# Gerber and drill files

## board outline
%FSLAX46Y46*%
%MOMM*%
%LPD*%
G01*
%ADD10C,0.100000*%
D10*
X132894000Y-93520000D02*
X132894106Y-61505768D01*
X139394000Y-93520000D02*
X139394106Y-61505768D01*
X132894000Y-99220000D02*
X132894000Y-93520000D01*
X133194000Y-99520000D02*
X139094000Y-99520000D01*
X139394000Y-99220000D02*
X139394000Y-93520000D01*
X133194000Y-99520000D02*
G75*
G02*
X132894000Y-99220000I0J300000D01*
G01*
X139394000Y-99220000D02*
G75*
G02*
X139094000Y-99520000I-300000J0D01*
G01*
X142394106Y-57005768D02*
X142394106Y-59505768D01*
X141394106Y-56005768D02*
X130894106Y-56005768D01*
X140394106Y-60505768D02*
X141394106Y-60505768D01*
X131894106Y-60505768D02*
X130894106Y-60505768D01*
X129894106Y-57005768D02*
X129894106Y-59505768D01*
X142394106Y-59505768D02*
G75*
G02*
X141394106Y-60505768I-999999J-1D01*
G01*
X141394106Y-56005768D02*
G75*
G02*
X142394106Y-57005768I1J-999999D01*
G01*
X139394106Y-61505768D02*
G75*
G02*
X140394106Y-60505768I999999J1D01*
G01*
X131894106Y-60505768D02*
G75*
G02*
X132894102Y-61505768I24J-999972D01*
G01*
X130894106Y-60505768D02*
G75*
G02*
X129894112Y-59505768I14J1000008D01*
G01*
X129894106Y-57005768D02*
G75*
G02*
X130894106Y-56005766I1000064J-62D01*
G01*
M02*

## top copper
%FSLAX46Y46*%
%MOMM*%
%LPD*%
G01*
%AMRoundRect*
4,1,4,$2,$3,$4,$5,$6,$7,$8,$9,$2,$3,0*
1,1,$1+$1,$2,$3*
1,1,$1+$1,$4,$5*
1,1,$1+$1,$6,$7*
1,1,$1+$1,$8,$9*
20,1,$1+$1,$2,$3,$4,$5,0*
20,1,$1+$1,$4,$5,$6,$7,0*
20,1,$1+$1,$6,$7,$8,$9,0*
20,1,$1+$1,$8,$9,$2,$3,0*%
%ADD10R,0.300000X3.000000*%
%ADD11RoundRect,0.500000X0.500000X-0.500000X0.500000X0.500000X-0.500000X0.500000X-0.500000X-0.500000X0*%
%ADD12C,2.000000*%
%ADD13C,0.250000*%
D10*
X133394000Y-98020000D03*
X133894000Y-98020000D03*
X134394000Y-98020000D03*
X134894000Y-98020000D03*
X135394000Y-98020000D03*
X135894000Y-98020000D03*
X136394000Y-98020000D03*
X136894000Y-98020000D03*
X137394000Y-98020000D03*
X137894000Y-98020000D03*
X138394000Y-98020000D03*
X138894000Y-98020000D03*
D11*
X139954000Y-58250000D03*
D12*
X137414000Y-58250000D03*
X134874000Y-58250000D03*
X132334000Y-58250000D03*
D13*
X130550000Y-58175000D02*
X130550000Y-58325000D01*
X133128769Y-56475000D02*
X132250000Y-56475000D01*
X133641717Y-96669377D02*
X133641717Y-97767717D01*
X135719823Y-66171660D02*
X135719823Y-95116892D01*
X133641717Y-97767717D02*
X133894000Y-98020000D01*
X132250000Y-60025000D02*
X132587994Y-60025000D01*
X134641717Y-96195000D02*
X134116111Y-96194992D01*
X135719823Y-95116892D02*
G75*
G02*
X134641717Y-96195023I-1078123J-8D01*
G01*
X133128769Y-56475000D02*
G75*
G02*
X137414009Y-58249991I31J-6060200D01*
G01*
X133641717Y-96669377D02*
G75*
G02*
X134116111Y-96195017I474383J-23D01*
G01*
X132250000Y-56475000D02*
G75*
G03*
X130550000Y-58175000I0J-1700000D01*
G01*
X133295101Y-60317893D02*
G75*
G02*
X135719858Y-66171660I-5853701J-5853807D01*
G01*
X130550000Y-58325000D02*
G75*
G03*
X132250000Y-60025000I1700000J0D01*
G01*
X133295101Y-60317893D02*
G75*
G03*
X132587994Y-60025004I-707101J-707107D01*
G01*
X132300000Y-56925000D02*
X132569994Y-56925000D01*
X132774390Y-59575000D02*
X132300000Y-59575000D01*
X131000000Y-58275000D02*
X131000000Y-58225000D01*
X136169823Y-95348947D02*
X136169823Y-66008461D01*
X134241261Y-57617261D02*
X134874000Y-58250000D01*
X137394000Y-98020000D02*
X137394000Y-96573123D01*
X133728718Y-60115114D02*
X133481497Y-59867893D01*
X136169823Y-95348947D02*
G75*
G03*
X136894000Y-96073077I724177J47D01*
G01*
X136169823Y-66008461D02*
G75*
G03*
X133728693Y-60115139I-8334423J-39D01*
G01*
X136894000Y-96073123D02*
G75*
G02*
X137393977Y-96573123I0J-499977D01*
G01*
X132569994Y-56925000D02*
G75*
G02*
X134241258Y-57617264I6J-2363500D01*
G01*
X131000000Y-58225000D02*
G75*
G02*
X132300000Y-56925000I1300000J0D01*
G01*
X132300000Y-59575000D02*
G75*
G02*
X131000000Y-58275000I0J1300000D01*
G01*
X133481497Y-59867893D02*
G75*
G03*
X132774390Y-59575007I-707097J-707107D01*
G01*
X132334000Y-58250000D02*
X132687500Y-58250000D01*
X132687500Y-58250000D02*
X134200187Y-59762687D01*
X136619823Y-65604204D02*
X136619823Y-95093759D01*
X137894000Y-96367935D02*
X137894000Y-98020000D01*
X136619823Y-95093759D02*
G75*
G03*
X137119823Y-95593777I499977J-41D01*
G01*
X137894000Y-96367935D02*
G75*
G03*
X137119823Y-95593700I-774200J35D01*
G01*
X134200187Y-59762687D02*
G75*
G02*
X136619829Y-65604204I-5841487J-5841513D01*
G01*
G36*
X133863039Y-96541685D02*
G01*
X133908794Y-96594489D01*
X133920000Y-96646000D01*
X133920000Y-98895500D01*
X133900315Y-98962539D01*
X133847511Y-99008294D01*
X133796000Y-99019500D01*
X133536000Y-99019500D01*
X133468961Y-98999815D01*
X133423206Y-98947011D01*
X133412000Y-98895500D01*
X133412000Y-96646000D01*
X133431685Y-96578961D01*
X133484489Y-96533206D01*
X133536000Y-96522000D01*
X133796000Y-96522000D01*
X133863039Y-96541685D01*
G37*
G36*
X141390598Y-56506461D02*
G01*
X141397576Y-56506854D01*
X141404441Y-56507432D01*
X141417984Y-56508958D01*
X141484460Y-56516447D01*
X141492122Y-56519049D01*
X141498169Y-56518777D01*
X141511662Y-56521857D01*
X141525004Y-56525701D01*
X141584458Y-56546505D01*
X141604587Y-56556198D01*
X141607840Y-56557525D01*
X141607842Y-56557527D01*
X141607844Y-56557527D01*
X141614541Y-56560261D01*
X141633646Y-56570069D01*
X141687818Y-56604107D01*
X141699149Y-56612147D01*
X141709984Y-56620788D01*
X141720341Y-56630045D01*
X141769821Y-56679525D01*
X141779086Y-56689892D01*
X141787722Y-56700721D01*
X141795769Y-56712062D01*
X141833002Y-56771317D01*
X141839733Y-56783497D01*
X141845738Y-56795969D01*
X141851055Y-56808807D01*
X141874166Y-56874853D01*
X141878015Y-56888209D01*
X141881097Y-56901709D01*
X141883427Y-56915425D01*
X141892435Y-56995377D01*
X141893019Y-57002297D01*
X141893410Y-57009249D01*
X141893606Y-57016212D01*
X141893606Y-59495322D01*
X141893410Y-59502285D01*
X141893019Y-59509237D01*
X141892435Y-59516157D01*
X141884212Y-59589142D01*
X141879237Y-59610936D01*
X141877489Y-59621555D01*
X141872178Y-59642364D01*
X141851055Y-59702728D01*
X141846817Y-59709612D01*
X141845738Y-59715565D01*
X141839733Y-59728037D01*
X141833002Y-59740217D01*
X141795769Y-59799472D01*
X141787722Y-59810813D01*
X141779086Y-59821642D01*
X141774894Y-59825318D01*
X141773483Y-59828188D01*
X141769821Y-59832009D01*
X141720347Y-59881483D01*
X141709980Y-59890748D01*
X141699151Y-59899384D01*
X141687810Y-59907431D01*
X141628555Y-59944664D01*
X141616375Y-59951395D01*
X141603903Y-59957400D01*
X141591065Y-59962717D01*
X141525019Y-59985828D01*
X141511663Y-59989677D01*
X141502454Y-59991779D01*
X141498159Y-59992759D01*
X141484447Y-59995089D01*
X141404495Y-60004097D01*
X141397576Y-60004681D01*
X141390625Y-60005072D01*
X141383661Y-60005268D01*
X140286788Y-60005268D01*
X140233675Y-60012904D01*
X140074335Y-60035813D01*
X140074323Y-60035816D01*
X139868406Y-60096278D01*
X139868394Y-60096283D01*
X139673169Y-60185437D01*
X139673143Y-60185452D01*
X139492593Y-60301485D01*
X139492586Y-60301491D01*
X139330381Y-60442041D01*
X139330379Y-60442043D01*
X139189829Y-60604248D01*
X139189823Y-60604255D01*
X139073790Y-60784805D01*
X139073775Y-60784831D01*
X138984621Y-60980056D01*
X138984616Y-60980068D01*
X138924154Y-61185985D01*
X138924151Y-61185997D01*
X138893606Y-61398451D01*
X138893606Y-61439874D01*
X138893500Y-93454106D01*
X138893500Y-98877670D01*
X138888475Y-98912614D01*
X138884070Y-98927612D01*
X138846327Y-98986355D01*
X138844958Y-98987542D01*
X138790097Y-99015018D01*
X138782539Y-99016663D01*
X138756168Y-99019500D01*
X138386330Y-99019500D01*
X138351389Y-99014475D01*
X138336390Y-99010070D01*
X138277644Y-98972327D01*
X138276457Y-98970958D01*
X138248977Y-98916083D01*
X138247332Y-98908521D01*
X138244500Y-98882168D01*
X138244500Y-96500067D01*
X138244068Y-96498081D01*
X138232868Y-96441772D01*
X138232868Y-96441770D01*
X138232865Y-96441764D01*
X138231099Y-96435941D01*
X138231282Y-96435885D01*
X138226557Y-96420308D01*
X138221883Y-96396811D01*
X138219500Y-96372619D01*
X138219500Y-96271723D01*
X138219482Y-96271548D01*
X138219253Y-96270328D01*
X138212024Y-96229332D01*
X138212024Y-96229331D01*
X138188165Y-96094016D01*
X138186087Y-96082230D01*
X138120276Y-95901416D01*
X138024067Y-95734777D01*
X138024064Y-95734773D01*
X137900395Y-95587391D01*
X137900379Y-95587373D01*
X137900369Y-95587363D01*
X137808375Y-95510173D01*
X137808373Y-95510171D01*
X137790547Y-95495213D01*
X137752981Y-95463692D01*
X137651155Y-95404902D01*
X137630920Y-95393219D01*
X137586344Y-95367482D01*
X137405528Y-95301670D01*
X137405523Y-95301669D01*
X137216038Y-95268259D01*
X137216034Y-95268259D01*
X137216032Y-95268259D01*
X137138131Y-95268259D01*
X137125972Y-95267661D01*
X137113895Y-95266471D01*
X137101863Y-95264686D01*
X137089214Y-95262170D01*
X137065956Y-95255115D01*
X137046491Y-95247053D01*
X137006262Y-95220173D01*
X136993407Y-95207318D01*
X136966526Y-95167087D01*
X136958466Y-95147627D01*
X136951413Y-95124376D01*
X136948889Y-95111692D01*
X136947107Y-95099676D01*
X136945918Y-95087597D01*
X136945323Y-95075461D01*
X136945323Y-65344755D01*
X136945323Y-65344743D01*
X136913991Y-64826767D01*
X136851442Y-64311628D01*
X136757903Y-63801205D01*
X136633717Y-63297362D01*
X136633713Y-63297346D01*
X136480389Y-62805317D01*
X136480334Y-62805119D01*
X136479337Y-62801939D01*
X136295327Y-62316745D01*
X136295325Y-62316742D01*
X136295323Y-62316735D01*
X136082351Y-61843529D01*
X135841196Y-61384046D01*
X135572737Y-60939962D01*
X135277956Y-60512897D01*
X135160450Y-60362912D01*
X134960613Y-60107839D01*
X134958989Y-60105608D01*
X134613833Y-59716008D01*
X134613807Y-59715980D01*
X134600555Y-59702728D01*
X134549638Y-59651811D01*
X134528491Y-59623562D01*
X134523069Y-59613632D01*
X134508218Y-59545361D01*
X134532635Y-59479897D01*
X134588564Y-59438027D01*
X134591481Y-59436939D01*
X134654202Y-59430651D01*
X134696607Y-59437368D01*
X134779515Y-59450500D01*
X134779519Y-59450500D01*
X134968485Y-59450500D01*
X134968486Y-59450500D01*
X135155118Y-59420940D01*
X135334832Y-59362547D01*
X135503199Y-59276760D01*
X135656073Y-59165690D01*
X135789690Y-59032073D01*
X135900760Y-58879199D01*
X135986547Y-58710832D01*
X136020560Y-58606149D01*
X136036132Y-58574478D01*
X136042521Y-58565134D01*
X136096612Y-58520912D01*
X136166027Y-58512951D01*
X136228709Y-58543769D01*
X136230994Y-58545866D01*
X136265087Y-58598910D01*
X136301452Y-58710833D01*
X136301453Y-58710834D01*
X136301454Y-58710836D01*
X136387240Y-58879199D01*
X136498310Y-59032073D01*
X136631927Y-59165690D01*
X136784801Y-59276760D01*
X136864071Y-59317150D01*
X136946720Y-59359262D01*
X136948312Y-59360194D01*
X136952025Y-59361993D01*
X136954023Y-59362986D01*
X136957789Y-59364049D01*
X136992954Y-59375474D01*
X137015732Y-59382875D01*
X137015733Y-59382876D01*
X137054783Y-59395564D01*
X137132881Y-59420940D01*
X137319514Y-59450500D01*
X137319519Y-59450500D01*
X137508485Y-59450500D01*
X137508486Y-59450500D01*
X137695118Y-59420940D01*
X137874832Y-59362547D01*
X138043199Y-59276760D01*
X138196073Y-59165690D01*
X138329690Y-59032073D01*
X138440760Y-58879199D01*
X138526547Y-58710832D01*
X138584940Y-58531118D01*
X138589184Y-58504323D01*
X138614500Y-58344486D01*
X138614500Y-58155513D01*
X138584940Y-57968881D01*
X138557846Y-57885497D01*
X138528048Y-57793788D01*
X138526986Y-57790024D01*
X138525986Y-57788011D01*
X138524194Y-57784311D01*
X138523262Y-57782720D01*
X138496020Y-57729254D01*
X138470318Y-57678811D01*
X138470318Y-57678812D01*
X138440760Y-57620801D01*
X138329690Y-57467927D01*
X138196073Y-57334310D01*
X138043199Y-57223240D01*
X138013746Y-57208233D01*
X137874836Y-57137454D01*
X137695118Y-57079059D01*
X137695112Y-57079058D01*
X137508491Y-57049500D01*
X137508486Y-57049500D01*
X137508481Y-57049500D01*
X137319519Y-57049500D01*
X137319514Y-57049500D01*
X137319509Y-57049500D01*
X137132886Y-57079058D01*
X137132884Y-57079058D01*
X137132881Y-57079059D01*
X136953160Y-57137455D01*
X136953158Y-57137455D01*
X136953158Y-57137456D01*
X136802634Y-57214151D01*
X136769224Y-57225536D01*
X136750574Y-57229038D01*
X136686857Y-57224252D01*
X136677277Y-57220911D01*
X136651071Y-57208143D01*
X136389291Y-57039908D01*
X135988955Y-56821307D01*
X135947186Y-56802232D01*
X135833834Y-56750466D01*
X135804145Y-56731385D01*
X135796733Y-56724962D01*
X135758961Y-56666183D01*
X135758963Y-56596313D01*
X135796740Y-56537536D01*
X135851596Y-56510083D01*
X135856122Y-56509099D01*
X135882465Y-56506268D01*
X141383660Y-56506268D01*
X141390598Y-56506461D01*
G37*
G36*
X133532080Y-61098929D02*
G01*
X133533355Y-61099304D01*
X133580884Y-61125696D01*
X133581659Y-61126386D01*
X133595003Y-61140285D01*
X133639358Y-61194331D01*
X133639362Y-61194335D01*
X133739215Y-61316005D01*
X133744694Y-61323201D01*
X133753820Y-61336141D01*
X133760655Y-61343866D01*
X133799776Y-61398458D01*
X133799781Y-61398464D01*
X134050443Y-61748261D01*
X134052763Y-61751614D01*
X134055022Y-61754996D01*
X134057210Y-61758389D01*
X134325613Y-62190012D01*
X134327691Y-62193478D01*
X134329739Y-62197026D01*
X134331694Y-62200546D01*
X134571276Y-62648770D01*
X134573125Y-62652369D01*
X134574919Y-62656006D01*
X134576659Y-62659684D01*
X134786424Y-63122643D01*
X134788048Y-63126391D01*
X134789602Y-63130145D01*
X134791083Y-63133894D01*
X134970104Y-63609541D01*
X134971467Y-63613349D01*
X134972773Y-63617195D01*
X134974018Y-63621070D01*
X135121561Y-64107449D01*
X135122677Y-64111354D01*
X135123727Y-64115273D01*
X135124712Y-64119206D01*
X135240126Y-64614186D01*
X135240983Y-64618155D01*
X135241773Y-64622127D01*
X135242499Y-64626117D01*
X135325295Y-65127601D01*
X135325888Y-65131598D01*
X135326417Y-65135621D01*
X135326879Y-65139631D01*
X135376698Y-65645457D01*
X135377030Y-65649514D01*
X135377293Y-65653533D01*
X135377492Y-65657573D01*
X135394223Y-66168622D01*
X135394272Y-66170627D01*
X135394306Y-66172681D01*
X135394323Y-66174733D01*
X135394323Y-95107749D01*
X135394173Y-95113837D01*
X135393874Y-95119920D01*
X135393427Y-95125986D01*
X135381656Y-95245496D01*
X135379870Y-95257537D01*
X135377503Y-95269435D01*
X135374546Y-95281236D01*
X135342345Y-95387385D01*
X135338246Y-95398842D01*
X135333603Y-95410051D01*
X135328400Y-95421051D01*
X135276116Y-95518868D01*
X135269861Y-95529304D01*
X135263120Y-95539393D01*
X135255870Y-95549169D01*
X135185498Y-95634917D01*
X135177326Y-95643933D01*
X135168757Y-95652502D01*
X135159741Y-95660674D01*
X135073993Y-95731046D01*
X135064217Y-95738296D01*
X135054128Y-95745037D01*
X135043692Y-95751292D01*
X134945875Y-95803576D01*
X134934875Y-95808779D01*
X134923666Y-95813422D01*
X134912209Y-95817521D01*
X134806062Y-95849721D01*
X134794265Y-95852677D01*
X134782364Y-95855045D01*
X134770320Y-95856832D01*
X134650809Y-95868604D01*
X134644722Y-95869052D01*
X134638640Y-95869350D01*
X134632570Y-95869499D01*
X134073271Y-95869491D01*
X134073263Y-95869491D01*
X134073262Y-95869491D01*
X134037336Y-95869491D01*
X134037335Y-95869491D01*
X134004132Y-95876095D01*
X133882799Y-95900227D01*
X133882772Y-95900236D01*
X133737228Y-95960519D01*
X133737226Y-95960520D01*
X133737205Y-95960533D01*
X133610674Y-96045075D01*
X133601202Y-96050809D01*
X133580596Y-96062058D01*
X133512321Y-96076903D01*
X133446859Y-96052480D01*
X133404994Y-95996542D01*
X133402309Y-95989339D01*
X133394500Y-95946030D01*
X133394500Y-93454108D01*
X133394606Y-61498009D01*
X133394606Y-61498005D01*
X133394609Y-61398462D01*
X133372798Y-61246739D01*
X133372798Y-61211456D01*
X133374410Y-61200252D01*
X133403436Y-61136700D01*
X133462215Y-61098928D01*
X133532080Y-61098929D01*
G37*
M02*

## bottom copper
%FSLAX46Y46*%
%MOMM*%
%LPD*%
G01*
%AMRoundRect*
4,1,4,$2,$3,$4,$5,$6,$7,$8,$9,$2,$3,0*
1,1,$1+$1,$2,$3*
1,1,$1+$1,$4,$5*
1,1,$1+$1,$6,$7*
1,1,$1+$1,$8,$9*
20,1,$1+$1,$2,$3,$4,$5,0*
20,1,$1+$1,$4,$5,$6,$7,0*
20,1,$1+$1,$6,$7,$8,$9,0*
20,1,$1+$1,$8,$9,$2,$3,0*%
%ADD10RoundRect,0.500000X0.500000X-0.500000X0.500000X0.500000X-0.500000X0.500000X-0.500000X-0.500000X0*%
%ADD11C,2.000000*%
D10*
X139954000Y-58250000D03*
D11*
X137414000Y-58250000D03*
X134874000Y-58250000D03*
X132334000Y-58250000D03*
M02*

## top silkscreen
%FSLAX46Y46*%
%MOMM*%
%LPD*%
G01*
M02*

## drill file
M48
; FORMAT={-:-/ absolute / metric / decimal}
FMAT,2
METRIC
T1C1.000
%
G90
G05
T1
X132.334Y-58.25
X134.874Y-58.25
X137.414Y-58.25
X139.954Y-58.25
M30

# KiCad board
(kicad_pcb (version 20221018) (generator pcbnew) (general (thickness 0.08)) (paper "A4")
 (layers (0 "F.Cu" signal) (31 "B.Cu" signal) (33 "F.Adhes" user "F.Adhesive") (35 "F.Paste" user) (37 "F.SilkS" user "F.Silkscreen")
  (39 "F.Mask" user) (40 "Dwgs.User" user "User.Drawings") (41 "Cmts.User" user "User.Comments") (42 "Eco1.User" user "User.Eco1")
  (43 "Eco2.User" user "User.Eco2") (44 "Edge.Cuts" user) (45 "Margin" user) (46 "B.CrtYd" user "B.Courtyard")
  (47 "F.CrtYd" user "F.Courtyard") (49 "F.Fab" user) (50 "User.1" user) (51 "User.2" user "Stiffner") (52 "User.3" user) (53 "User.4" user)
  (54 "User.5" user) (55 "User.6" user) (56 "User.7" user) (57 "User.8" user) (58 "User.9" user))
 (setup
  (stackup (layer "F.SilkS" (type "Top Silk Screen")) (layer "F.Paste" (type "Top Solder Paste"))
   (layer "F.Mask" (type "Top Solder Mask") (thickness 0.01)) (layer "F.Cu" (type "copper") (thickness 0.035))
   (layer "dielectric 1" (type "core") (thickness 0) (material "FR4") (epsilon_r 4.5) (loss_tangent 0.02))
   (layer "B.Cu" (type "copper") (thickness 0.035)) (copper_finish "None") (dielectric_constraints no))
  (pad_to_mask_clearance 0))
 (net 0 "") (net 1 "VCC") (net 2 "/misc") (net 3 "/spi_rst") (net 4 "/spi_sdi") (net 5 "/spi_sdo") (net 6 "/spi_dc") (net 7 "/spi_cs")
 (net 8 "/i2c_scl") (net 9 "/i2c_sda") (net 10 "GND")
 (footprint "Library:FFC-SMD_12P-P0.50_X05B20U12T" (layer "F.Cu") (at 136.144 96.52)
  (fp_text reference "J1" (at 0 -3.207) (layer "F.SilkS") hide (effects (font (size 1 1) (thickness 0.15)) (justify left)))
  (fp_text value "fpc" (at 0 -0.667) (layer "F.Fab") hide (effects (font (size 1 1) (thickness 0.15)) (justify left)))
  (fp_line (start -3.25 2.7) (end -3.25 -3) (stroke (width 0.1) (type default)) (layer "Edge.Cuts"))
  (fp_line (start -2.95 3) (end 2.95 3) (stroke (width 0.1) (type default)) (layer "Edge.Cuts"))
  (fp_line (start 3.25 2.7) (end 3.25 -3) (stroke (width 0.1) (type default)) (layer "Edge.Cuts"))
  (fp_arc (start -2.95 3) (mid -3.162132 2.912132) (end -3.25 2.7) (stroke (width 0.1) (type default)) (layer "Edge.Cuts"))
  (fp_arc (start 3.25 2.7) (mid 3.162132 2.912132) (end 2.95 3) (stroke (width 0.1) (type default)) (layer "Edge.Cuts"))
  (pad "1" smd rect (at -2.75 1.5) (size 0.3 3) (layers "F.Cu" "F.Paste" "F.Mask") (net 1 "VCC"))
  (pad "2" smd rect (at -2.25 1.5) (size 0.3 3) (layers "F.Cu" "F.Paste" "F.Mask") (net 1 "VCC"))
  (pad "3" smd rect (at -1.75 1.5) (size 0.3 3) (layers "F.Cu" "F.Paste" "F.Mask") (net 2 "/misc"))
  (pad "4" smd rect (at -1.25 1.5) (size 0.3 3) (layers "F.Cu" "F.Paste" "F.Mask") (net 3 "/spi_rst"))
  (pad "5" smd rect (at -0.75 1.5) (size 0.3 3) (layers "F.Cu" "F.Paste" "F.Mask") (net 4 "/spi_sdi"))
  (pad "6" smd rect (at -0.25 1.5) (size 0.3 3) (layers "F.Cu" "F.Paste" "F.Mask") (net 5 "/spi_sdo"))
  (pad "7" smd rect (at 0.25 1.5) (size 0.3 3) (layers "F.Cu" "F.Paste" "F.Mask") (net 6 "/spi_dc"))
  (pad "8" smd rect (at 0.75 1.5) (size 0.3 3) (layers "F.Cu" "F.Paste" "F.Mask") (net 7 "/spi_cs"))
  (pad "9" smd rect (at 1.25 1.5) (size 0.3 3) (layers "F.Cu" "F.Paste" "F.Mask") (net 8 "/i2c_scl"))
  (pad "10" smd rect (at 1.75 1.5) (size 0.3 3) (layers "F.Cu" "F.Paste" "F.Mask") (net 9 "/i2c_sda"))
  (pad "11" smd rect (at 2.25 1.5) (size 0.3 3) (layers "F.Cu" "F.Paste" "F.Mask") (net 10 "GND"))
  (pad "12" smd rect (at 2.75 1.5) (size 0.3 3) (layers "F.Cu" "F.Paste" "F.Mask") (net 10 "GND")))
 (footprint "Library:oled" (layer "B.Cu") (at 136.144 58.25 180)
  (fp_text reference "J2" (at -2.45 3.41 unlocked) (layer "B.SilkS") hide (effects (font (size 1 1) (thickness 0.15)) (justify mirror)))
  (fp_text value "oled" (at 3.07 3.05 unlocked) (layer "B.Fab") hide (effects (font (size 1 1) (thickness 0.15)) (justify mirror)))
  (fp_line (start -6.250106 1.244232) (end -6.250106 -1.255768) (stroke (width 0.1) (type default)) (layer "Edge.Cuts"))
  (fp_line (start -5.250106 2.244232) (end 5.249894 2.244232) (stroke (width 0.1) (type default)) (layer "Edge.Cuts"))
  (fp_line (start -4.250106 -2.255768) (end -5.250106 -2.255768) (stroke (width 0.1) (type default)) (layer "Edge.Cuts"))
  (fp_line (start 4.249894 -2.255768) (end 5.249894 -2.255768) (stroke (width 0.1) (type default)) (layer "Edge.Cuts"))
  (fp_line (start 6.249894 1.244232) (end 6.249894 -1.255768) (stroke (width 0.1) (type default)) (layer "Edge.Cuts"))
  (fp_arc (start -6.250106 -1.255768) (mid -5.957213 -1.962875) (end -5.250106 -2.255768) (stroke (width 0.1) (type default))
   (layer "Edge.Cuts"))
  (fp_arc (start -5.250106 2.244232) (mid -5.957213 1.951339) (end -6.250106 1.244232) (stroke (width 0.1) (type default))
   (layer "Edge.Cuts"))
  (fp_arc (start -3.250106 -3.255768) (mid -3.542999 -2.548661) (end -4.250106 -2.255768) (stroke (width 0.1) (type default))
   (layer "Edge.Cuts"))
  (fp_arc (start 4.249894 -2.255768) (mid 3.542778 -2.548654) (end 3.249894 -3.255768) (stroke (width 0.1) (type default))
   (layer "Edge.Cuts"))
  (fp_arc (start 5.249894 -2.255768) (mid 5.956998 -1.962871) (end 6.249894 -1.255768) (stroke (width 0.1) (type default))
   (layer "Edge.Cuts"))
  (fp_arc (start 6.249894 1.244232) (mid 5.956989 1.951316) (end 5.249894 2.244232) (stroke (width 0.1) (type default)) (layer "Edge.Cuts"))
  (pad "1" thru_hole roundrect (at -3.81 0 90) (size 2 2) (drill 1) (layers "*.Cu" "*.Mask") (roundrect_rratio 0.25) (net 10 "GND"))
  (pad "2" thru_hole circle (at -1.27 0 90) (size 2 2) (drill 1) (layers "*.Cu" "*.Mask") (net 1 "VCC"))
  (pad "3" thru_hole circle (at 1.27 0 90) (size 2 2) (drill 1) (layers "*.Cu" "*.Mask") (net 8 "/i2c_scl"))
  (pad "4" thru_hole circle (at 3.81 0 90) (size 2 2) (drill 1) (layers "*.Cu" "*.Mask") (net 9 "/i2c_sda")))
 (gr_line (start 132.894 93.52) (end 132.894106 61.505768) (stroke (width 0.1) (type default)) (layer "Edge.Cuts"))
 (gr_line (start 139.394 93.52) (end 139.394106 61.505768) (stroke (width 0.1) (type default)) (layer "Edge.Cuts"))
 (segment (start 130.55 58.175) (end 130.55 58.325) (width 0.25) (layer "F.Cu") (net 1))
 (segment (start 133.128769 56.475) (end 132.25 56.475) (width 0.25) (layer "F.Cu") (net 1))
 (segment (start 133.641717 96.669377) (end 133.641717 97.767717) (width 0.25) (layer "F.Cu") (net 1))
 (segment (start 135.719823 66.17166) (end 135.719823 95.116892) (width 0.25) (layer "F.Cu") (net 1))
 (segment (start 133.641717 97.767717) (end 133.894 98.02) (width 0.25) (layer "F.Cu") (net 1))
 (segment (start 132.25 60.025) (end 132.587994 60.025) (width 0.25) (layer "F.Cu") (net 1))
 (segment (start 134.641717 96.195) (end 134.116111 96.194992) (width 0.25) (layer "F.Cu") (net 1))
 (arc (start 135.719823 95.116892) (mid 135.404052 95.879229) (end 134.641717 96.195) (width 0.25) (layer "F.Cu") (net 1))
 (arc (start 133.128769 56.475) (mid 135.447921 56.936308) (end 137.414 58.25) (width 0.25) (layer "F.Cu") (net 1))
 (arc (start 133.641717 96.669377) (mid 133.780664 96.333933) (end 134.116111 96.194992) (width 0.25) (layer "F.Cu") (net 1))
 (arc (start 132.25 56.475) (mid 131.047918 56.972918) (end 130.55 58.175) (width 0.25) (layer "F.Cu") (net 1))
 (arc (start 133.295101 60.317893) (mid 135.089664 63.003636) (end 135.719823 66.17166) (width 0.25) (layer "F.Cu") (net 1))
 (arc (start 130.55 58.325) (mid 131.047918 59.527082) (end 132.25 60.025) (width 0.25) (layer "F.Cu") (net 1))
 (arc (start 133.295101 60.317893) (mid 132.970678 60.10112) (end 132.587994 60.025) (width 0.25) (layer "F.Cu") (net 1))
 (segment (start 132.3 56.925) (end 132.569994 56.925) (width 0.25) (layer "F.Cu") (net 8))
 (segment (start 132.77439 59.575) (end 132.3 59.575) (width 0.25) (layer "F.Cu") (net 8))
 (segment (start 131 58.275) (end 131 58.225) (width 0.25) (layer "F.Cu") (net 8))
 (segment (start 136.169823 95.348947) (end 136.169823 66.008461) (width 0.25) (layer "F.Cu") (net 8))
 (segment (start 134.241261 57.617261) (end 134.874 58.25) (width 0.25) (layer "F.Cu") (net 8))
 (segment (start 137.394 98.02) (end 137.394 96.573123) (width 0.25) (layer "F.Cu") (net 8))
 (segment (start 133.728718 60.115114) (end 133.481497 59.867893) (width 0.25) (layer "F.Cu") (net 8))
 (arc (start 136.169823 95.348947) (mid 136.381929 95.861017) (end 136.894 96.073123) (width 0.25) (layer "F.Cu") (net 8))
 (arc (start 136.169823 66.008461) (mid 135.535401 62.819004) (end 133.728718 60.115114) (width 0.25) (layer "F.Cu") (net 8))
 (arc (start 136.894 96.073123) (mid 137.247553 96.21957) (end 137.394 96.573123) (width 0.25) (layer "F.Cu") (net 8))
 (arc (start 132.569994 56.925) (mid 133.474477 57.104913) (end 134.241261 57.617261) (width 0.25) (layer "F.Cu") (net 8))
 (arc (start 131 58.225) (mid 131.380761 57.305761) (end 132.3 56.925) (width 0.25) (layer "F.Cu") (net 8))
 (arc (start 132.3 59.575) (mid 131.380761 59.194239) (end 131 58.275) (width 0.25) (layer "F.Cu") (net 8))
 (arc (start 133.481497 59.867893) (mid 133.157074 59.65112) (end 132.77439 59.575) (width 0.25) (layer "F.Cu") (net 8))
 (segment (start 132.334 58.25) (end 132.6875 58.25) (width 0.25) (layer "F.Cu") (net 9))
 (segment (start 132.6875 58.25) (end 134.200187 59.762687) (width 0.25) (layer "F.Cu") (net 9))
 (segment (start 136.619823 65.604204) (end 136.619823 95.093759) (width 0.25) (layer "F.Cu") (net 9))
 (segment (start 137.894 96.367935) (end 137.894 98.02) (width 0.25) (layer "F.Cu") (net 9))
 (arc (start 136.619823 95.093759) (mid 136.76627 95.447312) (end 137.119823 95.593759) (width 0.25) (layer "F.Cu") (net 9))
 (arc (start 137.894 96.367935) (mid 137.667249 95.82051) (end 137.119823 95.593759) (width 0.25) (layer "F.Cu") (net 9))
 (arc (start 134.200187 59.762687) (mid 135.99098 62.442798) (end 136.619823 65.604204) (width 0.25) (layer "F.Cu") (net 9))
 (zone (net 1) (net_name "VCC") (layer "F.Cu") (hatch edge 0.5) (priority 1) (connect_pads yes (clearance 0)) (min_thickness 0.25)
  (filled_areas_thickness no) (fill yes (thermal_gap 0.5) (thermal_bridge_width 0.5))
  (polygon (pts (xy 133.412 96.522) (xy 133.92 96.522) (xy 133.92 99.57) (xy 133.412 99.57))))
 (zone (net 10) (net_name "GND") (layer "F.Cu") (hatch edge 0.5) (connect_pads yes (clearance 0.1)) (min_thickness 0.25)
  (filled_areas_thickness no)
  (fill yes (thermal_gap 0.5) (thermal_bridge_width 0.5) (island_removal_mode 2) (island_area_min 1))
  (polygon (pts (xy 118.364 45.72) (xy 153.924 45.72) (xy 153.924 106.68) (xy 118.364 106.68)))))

